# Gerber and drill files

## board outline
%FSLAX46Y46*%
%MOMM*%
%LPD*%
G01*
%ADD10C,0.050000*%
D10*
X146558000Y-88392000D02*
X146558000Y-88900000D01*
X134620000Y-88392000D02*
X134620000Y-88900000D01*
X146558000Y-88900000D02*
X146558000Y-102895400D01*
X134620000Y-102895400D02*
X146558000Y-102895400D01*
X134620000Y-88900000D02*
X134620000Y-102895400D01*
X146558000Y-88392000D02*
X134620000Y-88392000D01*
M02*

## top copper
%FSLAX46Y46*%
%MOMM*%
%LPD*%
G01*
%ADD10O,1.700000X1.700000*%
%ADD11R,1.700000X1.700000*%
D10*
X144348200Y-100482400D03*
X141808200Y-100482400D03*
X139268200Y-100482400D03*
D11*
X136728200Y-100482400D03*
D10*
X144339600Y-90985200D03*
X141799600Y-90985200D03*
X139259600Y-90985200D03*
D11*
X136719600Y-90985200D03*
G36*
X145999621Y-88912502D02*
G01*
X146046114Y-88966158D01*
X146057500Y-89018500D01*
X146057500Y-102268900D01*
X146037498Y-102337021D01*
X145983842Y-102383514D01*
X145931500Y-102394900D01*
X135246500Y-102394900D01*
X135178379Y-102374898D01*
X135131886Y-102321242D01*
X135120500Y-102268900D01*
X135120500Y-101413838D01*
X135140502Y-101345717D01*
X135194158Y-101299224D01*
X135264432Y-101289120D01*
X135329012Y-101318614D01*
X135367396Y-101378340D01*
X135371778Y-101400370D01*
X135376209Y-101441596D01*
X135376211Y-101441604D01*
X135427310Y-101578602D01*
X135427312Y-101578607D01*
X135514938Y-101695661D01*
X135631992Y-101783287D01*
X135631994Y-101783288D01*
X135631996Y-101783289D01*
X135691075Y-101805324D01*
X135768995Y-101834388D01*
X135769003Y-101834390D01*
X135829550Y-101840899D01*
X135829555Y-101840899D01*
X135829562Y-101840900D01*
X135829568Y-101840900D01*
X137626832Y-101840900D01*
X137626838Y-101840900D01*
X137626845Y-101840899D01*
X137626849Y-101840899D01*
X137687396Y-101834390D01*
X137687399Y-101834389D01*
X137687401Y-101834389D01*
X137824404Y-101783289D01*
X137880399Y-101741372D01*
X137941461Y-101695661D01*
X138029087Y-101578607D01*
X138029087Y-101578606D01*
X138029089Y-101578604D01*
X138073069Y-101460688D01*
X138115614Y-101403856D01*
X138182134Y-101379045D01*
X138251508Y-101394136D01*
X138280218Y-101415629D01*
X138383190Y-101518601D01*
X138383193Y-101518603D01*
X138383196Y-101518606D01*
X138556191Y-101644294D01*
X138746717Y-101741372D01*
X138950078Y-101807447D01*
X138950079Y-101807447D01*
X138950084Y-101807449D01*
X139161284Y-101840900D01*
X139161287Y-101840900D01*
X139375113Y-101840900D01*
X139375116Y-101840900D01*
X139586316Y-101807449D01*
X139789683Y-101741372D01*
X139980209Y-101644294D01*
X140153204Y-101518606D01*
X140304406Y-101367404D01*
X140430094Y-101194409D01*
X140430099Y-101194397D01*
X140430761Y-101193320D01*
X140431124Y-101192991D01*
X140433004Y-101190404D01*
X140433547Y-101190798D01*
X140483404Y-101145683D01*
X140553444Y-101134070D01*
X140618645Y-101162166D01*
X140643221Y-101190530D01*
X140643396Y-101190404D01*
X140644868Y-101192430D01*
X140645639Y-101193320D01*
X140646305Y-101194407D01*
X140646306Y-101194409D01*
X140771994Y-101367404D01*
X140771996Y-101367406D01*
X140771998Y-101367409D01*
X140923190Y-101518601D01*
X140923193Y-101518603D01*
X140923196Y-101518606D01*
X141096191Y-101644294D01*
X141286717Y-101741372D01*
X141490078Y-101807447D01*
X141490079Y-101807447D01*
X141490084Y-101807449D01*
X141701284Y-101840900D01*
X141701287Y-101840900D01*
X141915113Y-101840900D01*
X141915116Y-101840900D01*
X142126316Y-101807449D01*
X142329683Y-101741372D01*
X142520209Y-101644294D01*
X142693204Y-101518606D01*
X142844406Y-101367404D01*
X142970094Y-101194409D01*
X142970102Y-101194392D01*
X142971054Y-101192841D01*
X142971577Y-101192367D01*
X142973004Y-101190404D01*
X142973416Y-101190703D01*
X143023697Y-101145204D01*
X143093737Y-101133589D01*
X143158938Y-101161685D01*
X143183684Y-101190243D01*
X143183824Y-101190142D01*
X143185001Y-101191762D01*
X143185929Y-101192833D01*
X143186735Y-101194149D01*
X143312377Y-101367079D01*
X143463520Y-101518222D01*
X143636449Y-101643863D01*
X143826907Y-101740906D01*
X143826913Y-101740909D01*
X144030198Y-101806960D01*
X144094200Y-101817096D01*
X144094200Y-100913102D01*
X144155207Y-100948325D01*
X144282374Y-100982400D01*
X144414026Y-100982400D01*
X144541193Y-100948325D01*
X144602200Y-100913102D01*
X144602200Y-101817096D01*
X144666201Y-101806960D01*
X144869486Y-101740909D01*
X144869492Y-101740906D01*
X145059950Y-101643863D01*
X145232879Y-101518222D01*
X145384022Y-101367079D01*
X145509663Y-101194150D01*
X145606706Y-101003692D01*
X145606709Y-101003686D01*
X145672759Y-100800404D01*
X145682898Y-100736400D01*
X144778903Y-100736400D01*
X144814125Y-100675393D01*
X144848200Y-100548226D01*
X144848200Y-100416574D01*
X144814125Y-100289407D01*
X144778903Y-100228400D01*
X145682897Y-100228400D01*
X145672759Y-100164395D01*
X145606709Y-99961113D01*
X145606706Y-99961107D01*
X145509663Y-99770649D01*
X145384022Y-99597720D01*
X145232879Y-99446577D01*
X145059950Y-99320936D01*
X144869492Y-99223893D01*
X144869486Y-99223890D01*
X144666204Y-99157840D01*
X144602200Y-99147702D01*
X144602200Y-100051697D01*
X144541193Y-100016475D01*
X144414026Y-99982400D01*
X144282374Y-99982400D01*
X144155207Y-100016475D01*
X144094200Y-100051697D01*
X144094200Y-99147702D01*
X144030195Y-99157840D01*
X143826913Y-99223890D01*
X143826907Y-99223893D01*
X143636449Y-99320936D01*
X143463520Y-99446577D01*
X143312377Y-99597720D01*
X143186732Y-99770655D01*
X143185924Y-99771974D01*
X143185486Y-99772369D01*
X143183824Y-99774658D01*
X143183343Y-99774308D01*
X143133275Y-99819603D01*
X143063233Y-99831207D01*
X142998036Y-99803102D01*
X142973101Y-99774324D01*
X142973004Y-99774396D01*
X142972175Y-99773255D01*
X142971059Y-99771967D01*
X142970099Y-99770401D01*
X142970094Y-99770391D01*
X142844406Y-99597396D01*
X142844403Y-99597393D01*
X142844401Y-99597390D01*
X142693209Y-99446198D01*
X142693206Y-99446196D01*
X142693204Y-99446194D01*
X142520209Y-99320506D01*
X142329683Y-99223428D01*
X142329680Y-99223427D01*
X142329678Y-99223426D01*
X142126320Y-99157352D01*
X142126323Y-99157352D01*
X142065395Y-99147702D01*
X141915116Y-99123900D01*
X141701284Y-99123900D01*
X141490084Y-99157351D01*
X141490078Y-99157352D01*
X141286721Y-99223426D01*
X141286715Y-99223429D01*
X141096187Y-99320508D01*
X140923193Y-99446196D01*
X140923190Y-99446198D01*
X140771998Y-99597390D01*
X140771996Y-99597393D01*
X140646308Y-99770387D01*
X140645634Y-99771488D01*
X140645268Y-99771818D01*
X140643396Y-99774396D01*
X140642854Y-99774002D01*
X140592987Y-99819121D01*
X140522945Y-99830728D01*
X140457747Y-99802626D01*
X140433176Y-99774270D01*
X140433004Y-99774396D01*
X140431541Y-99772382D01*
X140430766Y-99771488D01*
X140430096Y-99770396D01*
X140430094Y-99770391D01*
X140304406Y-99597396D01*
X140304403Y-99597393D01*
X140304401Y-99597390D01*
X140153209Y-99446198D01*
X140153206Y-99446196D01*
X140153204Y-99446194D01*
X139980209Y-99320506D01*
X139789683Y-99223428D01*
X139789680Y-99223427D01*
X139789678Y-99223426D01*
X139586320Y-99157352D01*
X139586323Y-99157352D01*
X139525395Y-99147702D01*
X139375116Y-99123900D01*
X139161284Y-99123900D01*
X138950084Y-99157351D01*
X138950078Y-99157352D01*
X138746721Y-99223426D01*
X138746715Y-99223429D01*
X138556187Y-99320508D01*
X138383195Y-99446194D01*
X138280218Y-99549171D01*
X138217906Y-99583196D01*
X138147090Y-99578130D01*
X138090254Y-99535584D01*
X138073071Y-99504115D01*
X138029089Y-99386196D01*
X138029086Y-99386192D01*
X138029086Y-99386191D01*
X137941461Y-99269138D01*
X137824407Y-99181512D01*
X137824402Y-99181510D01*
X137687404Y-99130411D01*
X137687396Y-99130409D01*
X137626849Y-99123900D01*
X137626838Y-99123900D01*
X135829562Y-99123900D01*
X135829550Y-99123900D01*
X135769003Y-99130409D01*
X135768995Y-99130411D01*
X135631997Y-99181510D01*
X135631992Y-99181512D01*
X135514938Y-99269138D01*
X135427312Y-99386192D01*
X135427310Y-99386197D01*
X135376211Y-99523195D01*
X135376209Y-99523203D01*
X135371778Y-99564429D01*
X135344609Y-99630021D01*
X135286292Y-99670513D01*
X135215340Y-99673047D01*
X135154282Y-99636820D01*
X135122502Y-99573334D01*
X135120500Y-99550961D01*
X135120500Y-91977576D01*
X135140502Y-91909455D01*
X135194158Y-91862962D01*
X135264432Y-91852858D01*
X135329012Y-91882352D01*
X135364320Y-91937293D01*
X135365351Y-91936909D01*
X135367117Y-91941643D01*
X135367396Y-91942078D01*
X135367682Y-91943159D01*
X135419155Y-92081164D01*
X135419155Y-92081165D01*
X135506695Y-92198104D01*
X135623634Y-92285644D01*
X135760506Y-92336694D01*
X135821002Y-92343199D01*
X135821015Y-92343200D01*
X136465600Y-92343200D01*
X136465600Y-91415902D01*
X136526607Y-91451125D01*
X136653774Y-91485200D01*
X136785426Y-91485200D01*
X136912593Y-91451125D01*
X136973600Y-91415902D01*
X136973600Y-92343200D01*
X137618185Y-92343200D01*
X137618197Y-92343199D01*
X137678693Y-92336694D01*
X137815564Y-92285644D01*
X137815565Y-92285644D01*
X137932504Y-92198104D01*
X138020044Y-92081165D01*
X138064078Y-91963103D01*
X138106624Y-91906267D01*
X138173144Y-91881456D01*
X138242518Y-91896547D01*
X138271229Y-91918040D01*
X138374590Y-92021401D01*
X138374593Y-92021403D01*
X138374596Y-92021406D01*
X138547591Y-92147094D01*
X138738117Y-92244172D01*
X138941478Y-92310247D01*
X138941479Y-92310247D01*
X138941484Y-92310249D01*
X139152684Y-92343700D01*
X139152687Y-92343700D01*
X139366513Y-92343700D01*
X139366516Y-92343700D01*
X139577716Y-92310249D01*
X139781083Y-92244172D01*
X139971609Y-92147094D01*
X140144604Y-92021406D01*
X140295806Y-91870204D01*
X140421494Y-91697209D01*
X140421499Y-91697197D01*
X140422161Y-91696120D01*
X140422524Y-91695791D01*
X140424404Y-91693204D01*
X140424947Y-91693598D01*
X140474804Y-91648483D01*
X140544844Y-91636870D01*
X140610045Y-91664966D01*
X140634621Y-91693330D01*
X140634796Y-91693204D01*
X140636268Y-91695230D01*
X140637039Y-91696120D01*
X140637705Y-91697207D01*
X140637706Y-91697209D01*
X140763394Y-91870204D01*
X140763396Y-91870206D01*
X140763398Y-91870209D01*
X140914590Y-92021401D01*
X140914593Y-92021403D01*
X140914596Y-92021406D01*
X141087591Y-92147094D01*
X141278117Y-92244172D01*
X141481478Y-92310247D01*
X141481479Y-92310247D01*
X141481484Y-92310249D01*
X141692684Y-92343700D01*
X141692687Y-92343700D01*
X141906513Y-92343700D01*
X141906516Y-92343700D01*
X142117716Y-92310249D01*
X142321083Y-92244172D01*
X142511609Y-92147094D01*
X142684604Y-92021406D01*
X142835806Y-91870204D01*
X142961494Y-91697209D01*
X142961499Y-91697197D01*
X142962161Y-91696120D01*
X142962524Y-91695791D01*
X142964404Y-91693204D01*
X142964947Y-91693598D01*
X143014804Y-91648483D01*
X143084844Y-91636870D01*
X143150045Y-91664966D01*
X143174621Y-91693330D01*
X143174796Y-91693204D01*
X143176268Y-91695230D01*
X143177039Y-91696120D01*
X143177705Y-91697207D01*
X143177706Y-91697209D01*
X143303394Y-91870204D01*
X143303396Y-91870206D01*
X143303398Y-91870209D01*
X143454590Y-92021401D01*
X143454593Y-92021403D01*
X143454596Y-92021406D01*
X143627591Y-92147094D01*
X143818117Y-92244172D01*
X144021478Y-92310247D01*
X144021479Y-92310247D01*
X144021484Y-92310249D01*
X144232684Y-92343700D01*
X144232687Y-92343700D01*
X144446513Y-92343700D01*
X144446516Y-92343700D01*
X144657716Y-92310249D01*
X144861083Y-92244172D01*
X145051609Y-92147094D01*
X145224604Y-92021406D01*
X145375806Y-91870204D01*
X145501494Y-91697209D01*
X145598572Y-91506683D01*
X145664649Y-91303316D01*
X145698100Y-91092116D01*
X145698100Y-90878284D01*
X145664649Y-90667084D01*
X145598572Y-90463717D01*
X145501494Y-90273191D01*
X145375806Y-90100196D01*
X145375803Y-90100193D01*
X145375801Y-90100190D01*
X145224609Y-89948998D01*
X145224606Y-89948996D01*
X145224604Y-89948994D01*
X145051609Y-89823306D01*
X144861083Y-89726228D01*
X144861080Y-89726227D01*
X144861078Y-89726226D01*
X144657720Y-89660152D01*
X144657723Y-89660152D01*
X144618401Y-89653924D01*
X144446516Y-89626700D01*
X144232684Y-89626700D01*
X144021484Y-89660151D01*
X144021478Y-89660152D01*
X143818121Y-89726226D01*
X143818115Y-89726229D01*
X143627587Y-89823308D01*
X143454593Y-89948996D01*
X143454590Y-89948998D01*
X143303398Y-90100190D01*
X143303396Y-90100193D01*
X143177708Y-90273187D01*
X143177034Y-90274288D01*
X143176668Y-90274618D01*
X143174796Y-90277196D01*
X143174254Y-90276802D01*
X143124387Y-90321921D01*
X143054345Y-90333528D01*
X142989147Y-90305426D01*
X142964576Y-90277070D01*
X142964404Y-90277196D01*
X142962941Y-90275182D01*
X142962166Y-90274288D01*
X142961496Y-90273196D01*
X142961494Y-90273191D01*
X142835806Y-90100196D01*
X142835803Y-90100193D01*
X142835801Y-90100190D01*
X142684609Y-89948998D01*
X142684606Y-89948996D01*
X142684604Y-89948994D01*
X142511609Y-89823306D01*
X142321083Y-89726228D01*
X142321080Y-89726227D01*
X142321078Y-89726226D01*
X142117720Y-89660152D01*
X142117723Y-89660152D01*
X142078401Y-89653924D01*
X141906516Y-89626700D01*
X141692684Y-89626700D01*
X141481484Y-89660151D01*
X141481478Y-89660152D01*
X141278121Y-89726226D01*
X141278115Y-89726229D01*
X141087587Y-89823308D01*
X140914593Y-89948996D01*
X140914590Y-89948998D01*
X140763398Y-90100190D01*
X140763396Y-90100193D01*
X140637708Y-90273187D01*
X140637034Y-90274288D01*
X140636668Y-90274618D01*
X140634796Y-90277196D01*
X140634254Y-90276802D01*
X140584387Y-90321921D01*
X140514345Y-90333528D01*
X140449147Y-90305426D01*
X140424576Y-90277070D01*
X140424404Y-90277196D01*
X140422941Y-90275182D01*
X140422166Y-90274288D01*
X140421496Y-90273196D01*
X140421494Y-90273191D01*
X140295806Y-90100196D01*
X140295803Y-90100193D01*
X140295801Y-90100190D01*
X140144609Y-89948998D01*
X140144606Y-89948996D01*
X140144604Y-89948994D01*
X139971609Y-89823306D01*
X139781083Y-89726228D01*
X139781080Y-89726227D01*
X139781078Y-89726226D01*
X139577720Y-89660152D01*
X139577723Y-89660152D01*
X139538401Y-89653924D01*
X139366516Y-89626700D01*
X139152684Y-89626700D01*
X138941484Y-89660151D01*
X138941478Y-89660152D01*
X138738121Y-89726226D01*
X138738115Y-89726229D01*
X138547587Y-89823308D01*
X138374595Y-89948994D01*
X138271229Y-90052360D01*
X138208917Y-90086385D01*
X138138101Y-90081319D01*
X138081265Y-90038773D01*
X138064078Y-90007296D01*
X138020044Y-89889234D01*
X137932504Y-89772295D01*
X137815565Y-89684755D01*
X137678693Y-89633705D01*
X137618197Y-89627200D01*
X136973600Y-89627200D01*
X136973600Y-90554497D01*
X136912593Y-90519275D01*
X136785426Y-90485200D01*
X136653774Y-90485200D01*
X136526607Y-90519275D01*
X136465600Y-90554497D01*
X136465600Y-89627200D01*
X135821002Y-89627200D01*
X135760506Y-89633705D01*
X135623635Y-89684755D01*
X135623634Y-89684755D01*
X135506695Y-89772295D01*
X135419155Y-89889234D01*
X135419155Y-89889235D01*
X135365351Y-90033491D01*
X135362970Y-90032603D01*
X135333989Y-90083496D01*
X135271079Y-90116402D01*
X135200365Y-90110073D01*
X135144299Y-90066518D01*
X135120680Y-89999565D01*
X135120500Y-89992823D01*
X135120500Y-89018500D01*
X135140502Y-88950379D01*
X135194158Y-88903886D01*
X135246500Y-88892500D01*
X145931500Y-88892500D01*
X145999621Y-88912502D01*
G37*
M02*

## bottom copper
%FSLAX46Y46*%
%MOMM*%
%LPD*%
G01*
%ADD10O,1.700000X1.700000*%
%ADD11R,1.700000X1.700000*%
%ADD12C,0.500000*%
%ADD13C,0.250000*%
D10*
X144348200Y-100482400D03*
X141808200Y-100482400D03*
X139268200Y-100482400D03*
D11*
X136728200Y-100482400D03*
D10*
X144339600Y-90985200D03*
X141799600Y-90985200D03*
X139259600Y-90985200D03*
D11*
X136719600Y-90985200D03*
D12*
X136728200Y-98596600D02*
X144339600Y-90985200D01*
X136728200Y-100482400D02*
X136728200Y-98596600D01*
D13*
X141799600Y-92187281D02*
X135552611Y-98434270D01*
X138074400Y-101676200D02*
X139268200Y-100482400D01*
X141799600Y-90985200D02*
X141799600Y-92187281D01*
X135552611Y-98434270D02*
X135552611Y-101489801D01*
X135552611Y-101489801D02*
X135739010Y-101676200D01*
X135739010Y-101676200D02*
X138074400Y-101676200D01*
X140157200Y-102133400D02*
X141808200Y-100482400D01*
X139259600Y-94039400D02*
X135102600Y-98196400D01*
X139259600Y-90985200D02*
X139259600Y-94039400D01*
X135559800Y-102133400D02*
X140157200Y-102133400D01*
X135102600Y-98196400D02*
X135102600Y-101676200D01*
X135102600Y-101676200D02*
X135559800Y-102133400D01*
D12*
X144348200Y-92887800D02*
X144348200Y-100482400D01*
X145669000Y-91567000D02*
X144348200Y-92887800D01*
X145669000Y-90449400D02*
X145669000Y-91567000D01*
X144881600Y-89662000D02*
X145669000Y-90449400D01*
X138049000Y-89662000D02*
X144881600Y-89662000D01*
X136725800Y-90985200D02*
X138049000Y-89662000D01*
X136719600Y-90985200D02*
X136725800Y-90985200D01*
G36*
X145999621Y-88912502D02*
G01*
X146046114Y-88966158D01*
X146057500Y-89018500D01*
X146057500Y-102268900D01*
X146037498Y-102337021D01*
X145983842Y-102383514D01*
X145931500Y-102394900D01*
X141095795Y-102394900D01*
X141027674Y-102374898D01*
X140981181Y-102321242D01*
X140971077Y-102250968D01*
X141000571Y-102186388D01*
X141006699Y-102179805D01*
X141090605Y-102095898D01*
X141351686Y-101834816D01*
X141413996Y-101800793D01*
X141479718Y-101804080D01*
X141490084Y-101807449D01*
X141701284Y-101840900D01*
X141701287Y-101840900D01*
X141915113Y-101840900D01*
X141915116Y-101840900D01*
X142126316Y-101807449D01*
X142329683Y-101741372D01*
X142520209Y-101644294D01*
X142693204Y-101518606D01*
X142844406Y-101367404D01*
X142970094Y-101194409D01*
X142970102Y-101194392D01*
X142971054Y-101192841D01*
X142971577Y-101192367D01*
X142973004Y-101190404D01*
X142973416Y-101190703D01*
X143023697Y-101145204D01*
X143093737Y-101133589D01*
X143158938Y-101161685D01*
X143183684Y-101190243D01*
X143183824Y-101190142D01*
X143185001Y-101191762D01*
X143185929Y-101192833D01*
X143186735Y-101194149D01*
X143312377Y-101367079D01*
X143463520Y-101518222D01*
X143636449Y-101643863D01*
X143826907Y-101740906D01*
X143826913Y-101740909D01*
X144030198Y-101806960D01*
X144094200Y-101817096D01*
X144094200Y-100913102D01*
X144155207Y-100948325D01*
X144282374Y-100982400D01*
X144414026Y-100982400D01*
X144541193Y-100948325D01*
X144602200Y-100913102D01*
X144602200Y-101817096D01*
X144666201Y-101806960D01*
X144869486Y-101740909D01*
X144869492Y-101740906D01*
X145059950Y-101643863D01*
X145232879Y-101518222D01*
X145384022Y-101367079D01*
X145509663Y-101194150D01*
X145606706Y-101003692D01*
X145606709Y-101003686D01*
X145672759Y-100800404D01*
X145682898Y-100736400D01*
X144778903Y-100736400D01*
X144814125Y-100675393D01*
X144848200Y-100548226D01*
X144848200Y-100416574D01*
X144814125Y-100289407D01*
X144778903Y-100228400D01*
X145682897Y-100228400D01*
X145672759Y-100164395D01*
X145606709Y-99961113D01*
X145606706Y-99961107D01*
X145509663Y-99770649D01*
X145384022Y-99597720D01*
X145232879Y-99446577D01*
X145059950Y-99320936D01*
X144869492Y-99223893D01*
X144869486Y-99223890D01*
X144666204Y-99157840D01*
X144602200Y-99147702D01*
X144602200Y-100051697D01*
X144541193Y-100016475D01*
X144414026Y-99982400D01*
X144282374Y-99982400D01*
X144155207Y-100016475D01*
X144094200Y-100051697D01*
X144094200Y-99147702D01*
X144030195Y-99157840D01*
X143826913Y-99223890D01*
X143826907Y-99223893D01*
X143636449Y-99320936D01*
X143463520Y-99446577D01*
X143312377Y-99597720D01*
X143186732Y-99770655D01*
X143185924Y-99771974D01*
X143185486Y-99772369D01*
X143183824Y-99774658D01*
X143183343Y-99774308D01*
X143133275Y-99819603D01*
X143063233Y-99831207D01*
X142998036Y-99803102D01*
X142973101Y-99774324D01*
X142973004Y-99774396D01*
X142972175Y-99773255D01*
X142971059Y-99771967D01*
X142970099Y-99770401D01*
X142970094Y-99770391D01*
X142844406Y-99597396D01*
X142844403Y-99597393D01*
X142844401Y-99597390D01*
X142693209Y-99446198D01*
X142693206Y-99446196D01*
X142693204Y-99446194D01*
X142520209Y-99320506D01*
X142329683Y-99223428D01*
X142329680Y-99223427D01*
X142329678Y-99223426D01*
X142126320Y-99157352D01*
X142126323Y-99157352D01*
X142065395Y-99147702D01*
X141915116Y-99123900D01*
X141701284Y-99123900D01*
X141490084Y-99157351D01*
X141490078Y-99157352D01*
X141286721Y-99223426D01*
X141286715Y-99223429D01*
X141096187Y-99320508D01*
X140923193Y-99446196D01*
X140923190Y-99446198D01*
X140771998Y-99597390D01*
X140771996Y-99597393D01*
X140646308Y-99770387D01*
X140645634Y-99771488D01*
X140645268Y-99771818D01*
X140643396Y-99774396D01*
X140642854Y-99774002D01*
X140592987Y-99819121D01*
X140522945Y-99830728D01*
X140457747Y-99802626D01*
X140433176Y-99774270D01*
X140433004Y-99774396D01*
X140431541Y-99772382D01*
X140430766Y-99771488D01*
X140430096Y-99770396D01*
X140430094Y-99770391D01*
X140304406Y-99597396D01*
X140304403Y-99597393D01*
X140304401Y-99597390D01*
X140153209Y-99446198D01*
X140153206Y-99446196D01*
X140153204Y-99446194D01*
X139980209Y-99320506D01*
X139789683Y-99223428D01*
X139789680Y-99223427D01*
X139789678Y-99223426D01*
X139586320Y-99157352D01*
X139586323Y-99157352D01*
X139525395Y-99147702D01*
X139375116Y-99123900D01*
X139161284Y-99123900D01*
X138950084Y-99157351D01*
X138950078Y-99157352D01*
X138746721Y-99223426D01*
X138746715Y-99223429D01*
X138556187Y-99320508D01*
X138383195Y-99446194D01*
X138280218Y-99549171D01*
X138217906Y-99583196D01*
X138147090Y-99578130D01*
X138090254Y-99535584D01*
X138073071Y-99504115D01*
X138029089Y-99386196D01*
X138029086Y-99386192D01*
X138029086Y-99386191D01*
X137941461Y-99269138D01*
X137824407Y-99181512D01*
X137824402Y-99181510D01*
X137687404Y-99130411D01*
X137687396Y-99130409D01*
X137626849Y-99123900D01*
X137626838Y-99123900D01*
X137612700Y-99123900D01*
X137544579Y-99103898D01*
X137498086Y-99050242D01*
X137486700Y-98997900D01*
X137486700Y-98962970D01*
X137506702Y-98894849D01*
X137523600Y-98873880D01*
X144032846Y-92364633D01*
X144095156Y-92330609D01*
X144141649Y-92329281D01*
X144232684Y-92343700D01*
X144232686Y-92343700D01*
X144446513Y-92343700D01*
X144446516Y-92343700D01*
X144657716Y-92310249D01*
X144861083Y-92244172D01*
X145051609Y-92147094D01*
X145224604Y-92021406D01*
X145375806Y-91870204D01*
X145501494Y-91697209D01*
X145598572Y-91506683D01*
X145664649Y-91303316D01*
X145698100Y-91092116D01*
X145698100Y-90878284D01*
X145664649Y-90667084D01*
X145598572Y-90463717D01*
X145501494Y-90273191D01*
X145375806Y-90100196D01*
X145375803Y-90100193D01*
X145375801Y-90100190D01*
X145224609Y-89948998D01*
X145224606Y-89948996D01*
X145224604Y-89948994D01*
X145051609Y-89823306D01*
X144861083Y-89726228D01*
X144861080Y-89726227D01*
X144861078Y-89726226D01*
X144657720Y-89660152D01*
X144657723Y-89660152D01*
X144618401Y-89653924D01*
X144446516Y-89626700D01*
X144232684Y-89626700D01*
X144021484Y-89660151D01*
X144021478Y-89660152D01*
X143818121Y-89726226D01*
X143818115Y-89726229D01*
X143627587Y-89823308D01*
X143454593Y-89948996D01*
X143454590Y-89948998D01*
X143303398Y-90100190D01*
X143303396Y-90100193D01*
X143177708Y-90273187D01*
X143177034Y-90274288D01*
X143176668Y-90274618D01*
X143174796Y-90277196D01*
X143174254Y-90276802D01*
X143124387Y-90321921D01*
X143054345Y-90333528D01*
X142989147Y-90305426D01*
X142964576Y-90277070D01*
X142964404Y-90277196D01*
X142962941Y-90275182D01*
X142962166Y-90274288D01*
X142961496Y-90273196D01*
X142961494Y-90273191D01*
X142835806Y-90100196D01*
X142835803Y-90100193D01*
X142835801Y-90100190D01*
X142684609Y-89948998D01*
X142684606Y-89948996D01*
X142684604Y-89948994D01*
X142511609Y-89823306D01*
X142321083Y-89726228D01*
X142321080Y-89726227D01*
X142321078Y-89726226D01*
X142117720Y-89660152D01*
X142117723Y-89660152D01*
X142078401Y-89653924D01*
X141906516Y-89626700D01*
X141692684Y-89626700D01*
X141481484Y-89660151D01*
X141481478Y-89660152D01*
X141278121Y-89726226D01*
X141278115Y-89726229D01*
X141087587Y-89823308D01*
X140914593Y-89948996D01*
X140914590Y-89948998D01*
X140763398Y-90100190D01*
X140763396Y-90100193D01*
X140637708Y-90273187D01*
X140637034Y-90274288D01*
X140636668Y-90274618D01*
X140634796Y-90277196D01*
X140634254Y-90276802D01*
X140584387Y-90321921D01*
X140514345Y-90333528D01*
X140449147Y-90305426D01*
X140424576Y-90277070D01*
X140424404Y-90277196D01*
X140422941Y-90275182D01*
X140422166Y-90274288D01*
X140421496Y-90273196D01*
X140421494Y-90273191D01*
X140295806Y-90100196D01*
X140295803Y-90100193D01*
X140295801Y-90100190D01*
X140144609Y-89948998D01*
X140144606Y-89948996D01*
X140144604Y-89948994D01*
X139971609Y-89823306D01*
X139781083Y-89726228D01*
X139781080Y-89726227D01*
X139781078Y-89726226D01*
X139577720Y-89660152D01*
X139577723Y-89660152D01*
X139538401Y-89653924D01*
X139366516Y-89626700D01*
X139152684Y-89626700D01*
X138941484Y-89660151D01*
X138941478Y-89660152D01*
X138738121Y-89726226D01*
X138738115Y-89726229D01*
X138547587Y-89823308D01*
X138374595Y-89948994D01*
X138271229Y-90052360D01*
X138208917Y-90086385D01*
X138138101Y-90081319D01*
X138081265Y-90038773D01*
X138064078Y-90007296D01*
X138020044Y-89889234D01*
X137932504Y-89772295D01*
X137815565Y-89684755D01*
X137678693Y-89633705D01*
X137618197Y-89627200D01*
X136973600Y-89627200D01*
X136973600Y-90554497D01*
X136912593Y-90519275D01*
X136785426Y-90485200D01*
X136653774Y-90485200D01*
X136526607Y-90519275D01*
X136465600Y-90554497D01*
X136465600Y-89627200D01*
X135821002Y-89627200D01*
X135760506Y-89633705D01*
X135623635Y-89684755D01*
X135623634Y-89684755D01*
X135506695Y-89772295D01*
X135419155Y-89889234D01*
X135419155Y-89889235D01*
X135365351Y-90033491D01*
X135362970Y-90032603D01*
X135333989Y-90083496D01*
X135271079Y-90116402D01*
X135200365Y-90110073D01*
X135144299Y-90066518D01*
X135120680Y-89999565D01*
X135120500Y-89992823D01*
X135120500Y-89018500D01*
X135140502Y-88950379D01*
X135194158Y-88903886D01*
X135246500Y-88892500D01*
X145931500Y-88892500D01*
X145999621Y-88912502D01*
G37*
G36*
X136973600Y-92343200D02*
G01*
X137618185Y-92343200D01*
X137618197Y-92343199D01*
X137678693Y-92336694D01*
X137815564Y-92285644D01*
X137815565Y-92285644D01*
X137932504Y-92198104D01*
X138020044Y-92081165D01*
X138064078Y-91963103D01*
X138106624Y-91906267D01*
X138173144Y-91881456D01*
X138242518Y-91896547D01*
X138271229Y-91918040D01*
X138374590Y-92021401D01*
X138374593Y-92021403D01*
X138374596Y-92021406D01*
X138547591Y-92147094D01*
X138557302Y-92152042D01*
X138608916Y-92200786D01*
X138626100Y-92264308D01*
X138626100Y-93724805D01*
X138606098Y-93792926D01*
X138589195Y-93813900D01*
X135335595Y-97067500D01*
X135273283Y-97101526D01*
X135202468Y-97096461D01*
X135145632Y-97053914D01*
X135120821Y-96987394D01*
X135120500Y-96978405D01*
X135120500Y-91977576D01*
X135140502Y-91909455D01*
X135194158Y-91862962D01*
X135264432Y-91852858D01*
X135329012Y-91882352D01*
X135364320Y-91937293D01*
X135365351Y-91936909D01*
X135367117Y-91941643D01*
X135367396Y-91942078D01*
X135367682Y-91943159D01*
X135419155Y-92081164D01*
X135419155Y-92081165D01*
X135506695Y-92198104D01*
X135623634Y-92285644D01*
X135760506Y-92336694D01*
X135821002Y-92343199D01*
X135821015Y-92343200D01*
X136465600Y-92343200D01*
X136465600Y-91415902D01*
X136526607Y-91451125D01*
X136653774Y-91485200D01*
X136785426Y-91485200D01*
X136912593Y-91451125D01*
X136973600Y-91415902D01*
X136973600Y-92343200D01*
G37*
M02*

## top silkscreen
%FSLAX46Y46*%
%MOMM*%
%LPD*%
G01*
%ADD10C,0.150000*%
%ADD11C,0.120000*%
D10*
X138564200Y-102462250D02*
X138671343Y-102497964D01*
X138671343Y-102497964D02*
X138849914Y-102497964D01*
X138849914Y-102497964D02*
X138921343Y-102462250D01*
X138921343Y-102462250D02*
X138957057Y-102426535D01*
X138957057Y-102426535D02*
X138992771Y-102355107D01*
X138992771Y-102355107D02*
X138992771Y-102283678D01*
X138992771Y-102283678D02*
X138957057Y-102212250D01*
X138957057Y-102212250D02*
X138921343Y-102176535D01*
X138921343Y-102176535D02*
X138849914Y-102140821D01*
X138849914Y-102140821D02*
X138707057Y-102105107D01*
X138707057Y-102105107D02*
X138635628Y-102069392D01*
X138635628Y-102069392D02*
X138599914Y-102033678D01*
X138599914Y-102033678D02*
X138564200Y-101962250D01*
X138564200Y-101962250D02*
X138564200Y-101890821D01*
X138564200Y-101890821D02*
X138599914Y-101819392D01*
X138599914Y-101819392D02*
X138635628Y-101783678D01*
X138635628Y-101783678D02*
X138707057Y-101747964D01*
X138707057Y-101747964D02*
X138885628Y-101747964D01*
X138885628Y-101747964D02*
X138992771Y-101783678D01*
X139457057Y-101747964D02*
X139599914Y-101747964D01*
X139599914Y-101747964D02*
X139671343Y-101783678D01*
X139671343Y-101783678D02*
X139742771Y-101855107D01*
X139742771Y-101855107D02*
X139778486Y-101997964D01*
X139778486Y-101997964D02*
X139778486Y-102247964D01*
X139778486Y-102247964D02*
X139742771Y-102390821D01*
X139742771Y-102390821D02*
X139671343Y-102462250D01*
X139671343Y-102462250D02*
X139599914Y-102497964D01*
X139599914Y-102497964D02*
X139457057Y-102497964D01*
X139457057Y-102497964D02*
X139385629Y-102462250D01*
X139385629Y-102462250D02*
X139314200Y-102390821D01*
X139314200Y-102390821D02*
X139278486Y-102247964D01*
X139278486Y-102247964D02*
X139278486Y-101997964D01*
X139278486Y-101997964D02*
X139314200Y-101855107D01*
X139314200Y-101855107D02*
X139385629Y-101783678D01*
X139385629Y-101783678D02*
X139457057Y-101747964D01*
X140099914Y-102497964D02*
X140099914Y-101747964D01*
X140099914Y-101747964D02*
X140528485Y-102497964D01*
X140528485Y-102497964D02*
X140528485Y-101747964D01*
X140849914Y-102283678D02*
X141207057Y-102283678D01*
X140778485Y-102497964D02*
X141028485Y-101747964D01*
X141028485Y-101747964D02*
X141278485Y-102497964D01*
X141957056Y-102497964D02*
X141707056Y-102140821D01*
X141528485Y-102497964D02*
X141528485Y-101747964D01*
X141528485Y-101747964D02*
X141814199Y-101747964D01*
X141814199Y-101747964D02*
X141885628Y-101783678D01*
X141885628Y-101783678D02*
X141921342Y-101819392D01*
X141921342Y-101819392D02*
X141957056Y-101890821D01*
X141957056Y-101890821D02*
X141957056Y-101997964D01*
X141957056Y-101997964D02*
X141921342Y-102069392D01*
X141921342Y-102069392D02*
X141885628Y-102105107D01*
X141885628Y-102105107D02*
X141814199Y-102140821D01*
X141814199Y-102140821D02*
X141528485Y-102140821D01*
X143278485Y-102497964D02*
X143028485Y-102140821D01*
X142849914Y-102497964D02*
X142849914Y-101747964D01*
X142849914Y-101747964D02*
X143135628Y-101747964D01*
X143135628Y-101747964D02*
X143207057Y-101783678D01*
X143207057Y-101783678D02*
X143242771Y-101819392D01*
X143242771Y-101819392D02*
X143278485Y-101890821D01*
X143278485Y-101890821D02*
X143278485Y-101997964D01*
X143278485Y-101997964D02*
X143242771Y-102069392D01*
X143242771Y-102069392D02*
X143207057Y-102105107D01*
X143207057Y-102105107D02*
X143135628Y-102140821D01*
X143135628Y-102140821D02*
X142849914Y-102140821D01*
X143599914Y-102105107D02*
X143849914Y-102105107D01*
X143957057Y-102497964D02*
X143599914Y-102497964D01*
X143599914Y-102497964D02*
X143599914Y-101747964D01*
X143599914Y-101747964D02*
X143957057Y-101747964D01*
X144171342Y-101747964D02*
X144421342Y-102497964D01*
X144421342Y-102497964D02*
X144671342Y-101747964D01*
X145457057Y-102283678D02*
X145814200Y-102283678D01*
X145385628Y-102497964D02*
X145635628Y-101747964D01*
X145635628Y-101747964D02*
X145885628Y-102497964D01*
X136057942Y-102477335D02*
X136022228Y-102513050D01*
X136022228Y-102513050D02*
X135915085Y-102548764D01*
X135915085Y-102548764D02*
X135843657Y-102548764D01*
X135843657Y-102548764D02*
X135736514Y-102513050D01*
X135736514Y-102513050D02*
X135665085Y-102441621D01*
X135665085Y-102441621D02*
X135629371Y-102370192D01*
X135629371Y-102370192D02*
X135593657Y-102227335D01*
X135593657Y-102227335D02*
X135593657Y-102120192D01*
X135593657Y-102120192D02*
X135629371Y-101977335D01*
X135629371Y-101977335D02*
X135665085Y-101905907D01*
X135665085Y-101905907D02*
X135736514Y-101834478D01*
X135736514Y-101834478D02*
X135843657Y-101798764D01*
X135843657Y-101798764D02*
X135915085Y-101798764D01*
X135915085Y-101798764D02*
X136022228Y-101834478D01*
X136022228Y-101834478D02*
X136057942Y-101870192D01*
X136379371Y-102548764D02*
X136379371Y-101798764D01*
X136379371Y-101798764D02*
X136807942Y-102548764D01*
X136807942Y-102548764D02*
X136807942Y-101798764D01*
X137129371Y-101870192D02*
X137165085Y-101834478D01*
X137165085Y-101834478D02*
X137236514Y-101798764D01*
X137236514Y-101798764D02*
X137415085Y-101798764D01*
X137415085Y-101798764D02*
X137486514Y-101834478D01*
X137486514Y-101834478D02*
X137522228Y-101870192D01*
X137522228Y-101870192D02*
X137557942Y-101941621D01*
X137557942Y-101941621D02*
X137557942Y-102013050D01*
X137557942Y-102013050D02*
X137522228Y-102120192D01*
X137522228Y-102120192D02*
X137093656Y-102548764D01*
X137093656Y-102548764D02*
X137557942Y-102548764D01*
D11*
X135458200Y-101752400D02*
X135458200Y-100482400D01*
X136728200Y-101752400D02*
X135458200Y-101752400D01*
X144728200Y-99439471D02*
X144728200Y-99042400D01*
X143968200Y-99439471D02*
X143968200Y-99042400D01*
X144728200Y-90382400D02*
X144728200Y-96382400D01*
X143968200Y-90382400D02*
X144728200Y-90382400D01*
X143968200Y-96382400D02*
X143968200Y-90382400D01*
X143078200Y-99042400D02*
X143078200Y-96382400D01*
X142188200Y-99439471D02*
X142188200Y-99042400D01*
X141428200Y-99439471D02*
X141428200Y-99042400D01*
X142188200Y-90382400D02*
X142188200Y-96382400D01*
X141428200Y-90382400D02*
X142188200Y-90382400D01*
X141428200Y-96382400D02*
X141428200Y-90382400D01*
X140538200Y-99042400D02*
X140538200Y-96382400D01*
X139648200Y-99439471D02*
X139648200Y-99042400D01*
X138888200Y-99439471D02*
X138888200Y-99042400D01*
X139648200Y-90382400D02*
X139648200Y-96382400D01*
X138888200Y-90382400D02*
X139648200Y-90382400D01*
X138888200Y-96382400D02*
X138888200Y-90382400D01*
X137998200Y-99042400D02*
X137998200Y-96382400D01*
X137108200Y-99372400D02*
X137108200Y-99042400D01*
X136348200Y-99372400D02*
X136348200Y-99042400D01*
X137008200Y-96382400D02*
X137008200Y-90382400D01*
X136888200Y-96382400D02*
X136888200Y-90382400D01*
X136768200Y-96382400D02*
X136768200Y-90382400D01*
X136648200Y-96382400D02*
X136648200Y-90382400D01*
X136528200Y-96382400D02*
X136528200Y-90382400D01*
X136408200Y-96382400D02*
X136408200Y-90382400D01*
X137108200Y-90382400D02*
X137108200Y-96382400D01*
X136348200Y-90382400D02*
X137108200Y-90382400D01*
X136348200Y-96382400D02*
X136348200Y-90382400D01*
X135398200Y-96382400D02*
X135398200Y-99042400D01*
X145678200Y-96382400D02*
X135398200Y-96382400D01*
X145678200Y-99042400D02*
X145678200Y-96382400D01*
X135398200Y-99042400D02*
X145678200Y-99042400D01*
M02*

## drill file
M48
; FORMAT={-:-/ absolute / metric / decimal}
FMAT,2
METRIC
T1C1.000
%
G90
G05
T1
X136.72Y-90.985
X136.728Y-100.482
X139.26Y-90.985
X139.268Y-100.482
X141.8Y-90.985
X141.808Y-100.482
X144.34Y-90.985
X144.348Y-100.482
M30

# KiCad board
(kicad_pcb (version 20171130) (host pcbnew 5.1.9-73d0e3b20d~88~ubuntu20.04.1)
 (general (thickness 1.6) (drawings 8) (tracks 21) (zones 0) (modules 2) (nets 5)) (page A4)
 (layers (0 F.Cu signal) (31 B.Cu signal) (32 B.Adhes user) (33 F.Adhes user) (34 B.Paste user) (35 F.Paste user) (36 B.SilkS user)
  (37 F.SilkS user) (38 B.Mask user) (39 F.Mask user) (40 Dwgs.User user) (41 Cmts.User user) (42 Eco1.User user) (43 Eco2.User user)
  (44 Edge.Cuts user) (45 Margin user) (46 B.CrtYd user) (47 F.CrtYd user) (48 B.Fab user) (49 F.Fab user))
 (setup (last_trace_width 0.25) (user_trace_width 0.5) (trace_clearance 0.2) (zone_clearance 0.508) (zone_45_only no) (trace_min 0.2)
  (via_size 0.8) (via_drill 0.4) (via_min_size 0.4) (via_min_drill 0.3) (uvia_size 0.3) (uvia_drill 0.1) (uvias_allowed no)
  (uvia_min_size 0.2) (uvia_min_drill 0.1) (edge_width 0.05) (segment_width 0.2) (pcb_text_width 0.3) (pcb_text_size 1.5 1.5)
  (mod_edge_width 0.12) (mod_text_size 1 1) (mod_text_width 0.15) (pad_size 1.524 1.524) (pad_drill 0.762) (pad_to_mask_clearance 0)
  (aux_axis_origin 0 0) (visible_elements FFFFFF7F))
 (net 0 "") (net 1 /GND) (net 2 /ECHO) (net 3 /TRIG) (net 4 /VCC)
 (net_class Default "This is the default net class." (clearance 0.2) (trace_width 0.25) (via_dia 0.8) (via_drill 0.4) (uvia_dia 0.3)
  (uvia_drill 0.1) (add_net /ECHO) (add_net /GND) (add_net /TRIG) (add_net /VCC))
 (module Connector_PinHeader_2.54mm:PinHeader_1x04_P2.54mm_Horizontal (layer F.Cu) (at 136.7282 100.4824 90)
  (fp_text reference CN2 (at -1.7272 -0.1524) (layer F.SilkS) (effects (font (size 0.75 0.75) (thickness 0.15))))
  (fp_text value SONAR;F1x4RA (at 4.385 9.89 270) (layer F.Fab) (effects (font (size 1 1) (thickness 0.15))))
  (fp_line (start -1.27 -1.27) (end 0 -1.27) (layer F.SilkS) (width 0.12))
  (fp_line (start -1.27 0) (end -1.27 -1.27) (layer F.SilkS) (width 0.12))
  (fp_line (start 1.042929 8) (end 1.44 8) (layer F.SilkS) (width 0.12))
  (fp_line (start 1.042929 7.24) (end 1.44 7.24) (layer F.SilkS) (width 0.12))
  (fp_line (start 10.1 8) (end 4.1 8) (layer F.SilkS) (width 0.12))
  (fp_line (start 10.1 7.24) (end 10.1 8) (layer F.SilkS) (width 0.12))
  (fp_line (start 4.1 7.24) (end 10.1 7.24) (layer F.SilkS) (width 0.12))
  (fp_line (start 1.44 6.35) (end 4.1 6.35) (layer F.SilkS) (width 0.12))
  (fp_line (start 1.042929 5.46) (end 1.44 5.46) (layer F.SilkS) (width 0.12))
  (fp_line (start 1.042929 4.7) (end 1.44 4.7) (layer F.SilkS) (width 0.12))
  (fp_line (start 10.1 5.46) (end 4.1 5.46) (layer F.SilkS) (width 0.12))
  (fp_line (start 10.1 4.7) (end 10.1 5.46) (layer F.SilkS) (width 0.12))
  (fp_line (start 4.1 4.7) (end 10.1 4.7) (layer F.SilkS) (width 0.12))
  (fp_line (start 1.44 3.81) (end 4.1 3.81) (layer F.SilkS) (width 0.12))
  (fp_line (start 1.042929 2.92) (end 1.44 2.92) (layer F.SilkS) (width 0.12))
  (fp_line (start 1.042929 2.16) (end 1.44 2.16) (layer F.SilkS) (width 0.12))
  (fp_line (start 10.1 2.92) (end 4.1 2.92) (layer F.SilkS) (width 0.12))
  (fp_line (start 10.1 2.16) (end 10.1 2.92) (layer F.SilkS) (width 0.12))
  (fp_line (start 4.1 2.16) (end 10.1 2.16) (layer F.SilkS) (width 0.12))
  (fp_line (start 1.44 1.27) (end 4.1 1.27) (layer F.SilkS) (width 0.12))
  (fp_line (start 1.11 0.38) (end 1.44 0.38) (layer F.SilkS) (width 0.12))
  (fp_line (start 1.11 -0.38) (end 1.44 -0.38) (layer F.SilkS) (width 0.12))
  (fp_line (start 4.1 0.28) (end 10.1 0.28) (layer F.SilkS) (width 0.12))
  (fp_line (start 4.1 0.16) (end 10.1 0.16) (layer F.SilkS) (width 0.12))
  (fp_line (start 4.1 0.04) (end 10.1 0.04) (layer F.SilkS) (width 0.12))
  (fp_line (start 4.1 -0.08) (end 10.1 -0.08) (layer F.SilkS) (width 0.12))
  (fp_line (start 4.1 -0.2) (end 10.1 -0.2) (layer F.SilkS) (width 0.12))
  (fp_line (start 4.1 -0.32) (end 10.1 -0.32) (layer F.SilkS) (width 0.12))
  (fp_line (start 10.1 0.38) (end 4.1 0.38) (layer F.SilkS) (width 0.12))
  (fp_line (start 10.1 -0.38) (end 10.1 0.38) (layer F.SilkS) (width 0.12))
  (fp_line (start 4.1 -0.38) (end 10.1 -0.38) (layer F.SilkS) (width 0.12))
  (fp_line (start 4.1 -1.33) (end 1.44 -1.33) (layer F.SilkS) (width 0.12))
  (fp_line (start 4.1 8.95) (end 4.1 -1.33) (layer F.SilkS) (width 0.12))
  (fp_line (start 1.44 8.95) (end 4.1 8.95) (layer F.SilkS) (width 0.12))
  (fp_line (start 1.44 -1.33) (end 1.44 8.95) (layer F.SilkS) (width 0.12))
  (pad 4 thru_hole oval (at 0 7.62 90) (size 1.7 1.7) (drill 1) (layers *.Cu *.Mask) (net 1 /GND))
  (pad 3 thru_hole oval (at 0 5.08 90) (size 1.7 1.7) (drill 1) (layers *.Cu *.Mask) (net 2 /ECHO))
  (pad 2 thru_hole oval (at 0 2.54 90) (size 1.7 1.7) (drill 1) (layers *.Cu *.Mask) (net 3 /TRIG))
  (pad 1 thru_hole rect (at 0 0 90) (size 1.7 1.7) (drill 1) (layers *.Cu *.Mask) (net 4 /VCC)))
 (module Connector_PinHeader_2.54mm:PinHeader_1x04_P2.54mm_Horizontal (layer B.Cu) (at 136.7196 90.9852 270)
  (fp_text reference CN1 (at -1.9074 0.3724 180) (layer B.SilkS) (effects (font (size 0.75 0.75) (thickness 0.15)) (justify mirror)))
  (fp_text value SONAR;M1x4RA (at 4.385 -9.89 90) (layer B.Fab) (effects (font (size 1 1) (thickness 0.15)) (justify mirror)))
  (pad 4 thru_hole oval (at 0 -7.62 270) (size 1.7 1.7) (drill 1) (layers *.Cu *.Mask) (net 4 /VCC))
  (pad 3 thru_hole oval (at 0 -5.08 270) (size 1.7 1.7) (drill 1) (layers *.Cu *.Mask) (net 3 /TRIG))
  (pad 2 thru_hole oval (at 0 -2.54 270) (size 1.7 1.7) (drill 1) (layers *.Cu *.Mask) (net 2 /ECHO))
  (pad 1 thru_hole rect (at 0 0 270) (size 1.7 1.7) (drill 1) (layers *.Cu *.Mask) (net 1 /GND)))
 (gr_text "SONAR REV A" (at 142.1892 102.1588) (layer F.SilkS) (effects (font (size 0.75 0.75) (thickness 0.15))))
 (gr_line (start 146.558 88.392) (end 146.558 88.9) (layer Edge.Cuts) (width 0.05))
 (gr_line (start 134.62 88.392) (end 134.62 88.9) (layer Edge.Cuts) (width 0.05))
 (gr_line (start 146.558 88.9) (end 146.558 102.8954) (layer Edge.Cuts) (width 0.05))
 (gr_line (start 134.62 102.8954) (end 146.558 102.8954) (layer Edge.Cuts) (width 0.05))
 (gr_line (start 134.62 88.9) (end 134.62 102.8954) (layer Edge.Cuts) (width 0.05))
 (gr_line (start 146.558 88.392) (end 134.62 88.392) (layer Edge.Cuts) (width 0.05))
 (segment (start 136.7282 98.5966) (end 144.3396 90.9852) (width 0.5) (layer B.Cu) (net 4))
 (segment (start 136.7282 100.4824) (end 136.7282 98.5966) (width 0.5) (layer B.Cu) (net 4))
 (segment (start 141.7996 92.187281) (end 135.552611 98.43427) (width 0.25) (layer B.Cu) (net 3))
 (segment (start 138.0744 101.6762) (end 139.2682 100.4824) (width 0.25) (layer B.Cu) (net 3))
 (segment (start 141.7996 90.9852) (end 141.7996 92.187281) (width 0.25) (layer B.Cu) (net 3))
 (segment (start 135.552611 98.43427) (end 135.552611 101.489801) (width 0.25) (layer B.Cu) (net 3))
 (segment (start 135.552611 101.489801) (end 135.73901 101.6762) (width 0.25) (layer B.Cu) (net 3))
 (segment (start 135.73901 101.6762) (end 138.0744 101.6762) (width 0.25) (layer B.Cu) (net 3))
 (segment (start 140.1572 102.1334) (end 141.8082 100.4824) (width 0.25) (layer B.Cu) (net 2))
 (segment (start 139.2596 94.0394) (end 135.1026 98.1964) (width 0.25) (layer B.Cu) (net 2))
 (segment (start 139.2596 90.9852) (end 139.2596 94.0394) (width 0.25) (layer B.Cu) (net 2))
 (segment (start 135.5598 102.1334) (end 140.1572 102.1334) (width 0.25) (layer B.Cu) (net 2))
 (segment (start 135.1026 98.1964) (end 135.1026 101.6762) (width 0.25) (layer B.Cu) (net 2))
 (segment (start 135.1026 101.6762) (end 135.5598 102.1334) (width 0.25) (layer B.Cu) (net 2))
 (segment (start 144.3482 92.8878) (end 144.3482 100.4824) (width 0.5) (layer B.Cu) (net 1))
 (segment (start 145.669 91.567) (end 144.3482 92.8878) (width 0.5) (layer B.Cu) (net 1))
 (segment (start 145.669 90.4494) (end 145.669 91.567) (width 0.5) (layer B.Cu) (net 1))
 (segment (start 144.8816 89.662) (end 145.669 90.4494) (width 0.5) (layer B.Cu) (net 1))
 (segment (start 138.049 89.662) (end 144.8816 89.662) (width 0.5) (layer B.Cu) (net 1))
 (segment (start 136.7258 90.9852) (end 138.049 89.662) (width 0.5) (layer B.Cu) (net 1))
 (segment (start 136.7196 90.9852) (end 136.7258 90.9852) (width 0.5) (layer B.Cu) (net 1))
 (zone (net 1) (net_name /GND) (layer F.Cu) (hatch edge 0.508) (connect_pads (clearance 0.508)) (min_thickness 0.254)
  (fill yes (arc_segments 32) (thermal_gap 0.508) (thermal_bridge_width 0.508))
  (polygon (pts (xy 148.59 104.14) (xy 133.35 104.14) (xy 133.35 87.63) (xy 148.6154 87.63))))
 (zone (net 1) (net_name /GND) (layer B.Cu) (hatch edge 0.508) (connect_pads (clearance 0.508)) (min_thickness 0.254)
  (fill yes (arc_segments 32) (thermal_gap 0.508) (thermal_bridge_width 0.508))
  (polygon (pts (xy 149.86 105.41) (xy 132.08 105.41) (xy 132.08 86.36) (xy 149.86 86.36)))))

